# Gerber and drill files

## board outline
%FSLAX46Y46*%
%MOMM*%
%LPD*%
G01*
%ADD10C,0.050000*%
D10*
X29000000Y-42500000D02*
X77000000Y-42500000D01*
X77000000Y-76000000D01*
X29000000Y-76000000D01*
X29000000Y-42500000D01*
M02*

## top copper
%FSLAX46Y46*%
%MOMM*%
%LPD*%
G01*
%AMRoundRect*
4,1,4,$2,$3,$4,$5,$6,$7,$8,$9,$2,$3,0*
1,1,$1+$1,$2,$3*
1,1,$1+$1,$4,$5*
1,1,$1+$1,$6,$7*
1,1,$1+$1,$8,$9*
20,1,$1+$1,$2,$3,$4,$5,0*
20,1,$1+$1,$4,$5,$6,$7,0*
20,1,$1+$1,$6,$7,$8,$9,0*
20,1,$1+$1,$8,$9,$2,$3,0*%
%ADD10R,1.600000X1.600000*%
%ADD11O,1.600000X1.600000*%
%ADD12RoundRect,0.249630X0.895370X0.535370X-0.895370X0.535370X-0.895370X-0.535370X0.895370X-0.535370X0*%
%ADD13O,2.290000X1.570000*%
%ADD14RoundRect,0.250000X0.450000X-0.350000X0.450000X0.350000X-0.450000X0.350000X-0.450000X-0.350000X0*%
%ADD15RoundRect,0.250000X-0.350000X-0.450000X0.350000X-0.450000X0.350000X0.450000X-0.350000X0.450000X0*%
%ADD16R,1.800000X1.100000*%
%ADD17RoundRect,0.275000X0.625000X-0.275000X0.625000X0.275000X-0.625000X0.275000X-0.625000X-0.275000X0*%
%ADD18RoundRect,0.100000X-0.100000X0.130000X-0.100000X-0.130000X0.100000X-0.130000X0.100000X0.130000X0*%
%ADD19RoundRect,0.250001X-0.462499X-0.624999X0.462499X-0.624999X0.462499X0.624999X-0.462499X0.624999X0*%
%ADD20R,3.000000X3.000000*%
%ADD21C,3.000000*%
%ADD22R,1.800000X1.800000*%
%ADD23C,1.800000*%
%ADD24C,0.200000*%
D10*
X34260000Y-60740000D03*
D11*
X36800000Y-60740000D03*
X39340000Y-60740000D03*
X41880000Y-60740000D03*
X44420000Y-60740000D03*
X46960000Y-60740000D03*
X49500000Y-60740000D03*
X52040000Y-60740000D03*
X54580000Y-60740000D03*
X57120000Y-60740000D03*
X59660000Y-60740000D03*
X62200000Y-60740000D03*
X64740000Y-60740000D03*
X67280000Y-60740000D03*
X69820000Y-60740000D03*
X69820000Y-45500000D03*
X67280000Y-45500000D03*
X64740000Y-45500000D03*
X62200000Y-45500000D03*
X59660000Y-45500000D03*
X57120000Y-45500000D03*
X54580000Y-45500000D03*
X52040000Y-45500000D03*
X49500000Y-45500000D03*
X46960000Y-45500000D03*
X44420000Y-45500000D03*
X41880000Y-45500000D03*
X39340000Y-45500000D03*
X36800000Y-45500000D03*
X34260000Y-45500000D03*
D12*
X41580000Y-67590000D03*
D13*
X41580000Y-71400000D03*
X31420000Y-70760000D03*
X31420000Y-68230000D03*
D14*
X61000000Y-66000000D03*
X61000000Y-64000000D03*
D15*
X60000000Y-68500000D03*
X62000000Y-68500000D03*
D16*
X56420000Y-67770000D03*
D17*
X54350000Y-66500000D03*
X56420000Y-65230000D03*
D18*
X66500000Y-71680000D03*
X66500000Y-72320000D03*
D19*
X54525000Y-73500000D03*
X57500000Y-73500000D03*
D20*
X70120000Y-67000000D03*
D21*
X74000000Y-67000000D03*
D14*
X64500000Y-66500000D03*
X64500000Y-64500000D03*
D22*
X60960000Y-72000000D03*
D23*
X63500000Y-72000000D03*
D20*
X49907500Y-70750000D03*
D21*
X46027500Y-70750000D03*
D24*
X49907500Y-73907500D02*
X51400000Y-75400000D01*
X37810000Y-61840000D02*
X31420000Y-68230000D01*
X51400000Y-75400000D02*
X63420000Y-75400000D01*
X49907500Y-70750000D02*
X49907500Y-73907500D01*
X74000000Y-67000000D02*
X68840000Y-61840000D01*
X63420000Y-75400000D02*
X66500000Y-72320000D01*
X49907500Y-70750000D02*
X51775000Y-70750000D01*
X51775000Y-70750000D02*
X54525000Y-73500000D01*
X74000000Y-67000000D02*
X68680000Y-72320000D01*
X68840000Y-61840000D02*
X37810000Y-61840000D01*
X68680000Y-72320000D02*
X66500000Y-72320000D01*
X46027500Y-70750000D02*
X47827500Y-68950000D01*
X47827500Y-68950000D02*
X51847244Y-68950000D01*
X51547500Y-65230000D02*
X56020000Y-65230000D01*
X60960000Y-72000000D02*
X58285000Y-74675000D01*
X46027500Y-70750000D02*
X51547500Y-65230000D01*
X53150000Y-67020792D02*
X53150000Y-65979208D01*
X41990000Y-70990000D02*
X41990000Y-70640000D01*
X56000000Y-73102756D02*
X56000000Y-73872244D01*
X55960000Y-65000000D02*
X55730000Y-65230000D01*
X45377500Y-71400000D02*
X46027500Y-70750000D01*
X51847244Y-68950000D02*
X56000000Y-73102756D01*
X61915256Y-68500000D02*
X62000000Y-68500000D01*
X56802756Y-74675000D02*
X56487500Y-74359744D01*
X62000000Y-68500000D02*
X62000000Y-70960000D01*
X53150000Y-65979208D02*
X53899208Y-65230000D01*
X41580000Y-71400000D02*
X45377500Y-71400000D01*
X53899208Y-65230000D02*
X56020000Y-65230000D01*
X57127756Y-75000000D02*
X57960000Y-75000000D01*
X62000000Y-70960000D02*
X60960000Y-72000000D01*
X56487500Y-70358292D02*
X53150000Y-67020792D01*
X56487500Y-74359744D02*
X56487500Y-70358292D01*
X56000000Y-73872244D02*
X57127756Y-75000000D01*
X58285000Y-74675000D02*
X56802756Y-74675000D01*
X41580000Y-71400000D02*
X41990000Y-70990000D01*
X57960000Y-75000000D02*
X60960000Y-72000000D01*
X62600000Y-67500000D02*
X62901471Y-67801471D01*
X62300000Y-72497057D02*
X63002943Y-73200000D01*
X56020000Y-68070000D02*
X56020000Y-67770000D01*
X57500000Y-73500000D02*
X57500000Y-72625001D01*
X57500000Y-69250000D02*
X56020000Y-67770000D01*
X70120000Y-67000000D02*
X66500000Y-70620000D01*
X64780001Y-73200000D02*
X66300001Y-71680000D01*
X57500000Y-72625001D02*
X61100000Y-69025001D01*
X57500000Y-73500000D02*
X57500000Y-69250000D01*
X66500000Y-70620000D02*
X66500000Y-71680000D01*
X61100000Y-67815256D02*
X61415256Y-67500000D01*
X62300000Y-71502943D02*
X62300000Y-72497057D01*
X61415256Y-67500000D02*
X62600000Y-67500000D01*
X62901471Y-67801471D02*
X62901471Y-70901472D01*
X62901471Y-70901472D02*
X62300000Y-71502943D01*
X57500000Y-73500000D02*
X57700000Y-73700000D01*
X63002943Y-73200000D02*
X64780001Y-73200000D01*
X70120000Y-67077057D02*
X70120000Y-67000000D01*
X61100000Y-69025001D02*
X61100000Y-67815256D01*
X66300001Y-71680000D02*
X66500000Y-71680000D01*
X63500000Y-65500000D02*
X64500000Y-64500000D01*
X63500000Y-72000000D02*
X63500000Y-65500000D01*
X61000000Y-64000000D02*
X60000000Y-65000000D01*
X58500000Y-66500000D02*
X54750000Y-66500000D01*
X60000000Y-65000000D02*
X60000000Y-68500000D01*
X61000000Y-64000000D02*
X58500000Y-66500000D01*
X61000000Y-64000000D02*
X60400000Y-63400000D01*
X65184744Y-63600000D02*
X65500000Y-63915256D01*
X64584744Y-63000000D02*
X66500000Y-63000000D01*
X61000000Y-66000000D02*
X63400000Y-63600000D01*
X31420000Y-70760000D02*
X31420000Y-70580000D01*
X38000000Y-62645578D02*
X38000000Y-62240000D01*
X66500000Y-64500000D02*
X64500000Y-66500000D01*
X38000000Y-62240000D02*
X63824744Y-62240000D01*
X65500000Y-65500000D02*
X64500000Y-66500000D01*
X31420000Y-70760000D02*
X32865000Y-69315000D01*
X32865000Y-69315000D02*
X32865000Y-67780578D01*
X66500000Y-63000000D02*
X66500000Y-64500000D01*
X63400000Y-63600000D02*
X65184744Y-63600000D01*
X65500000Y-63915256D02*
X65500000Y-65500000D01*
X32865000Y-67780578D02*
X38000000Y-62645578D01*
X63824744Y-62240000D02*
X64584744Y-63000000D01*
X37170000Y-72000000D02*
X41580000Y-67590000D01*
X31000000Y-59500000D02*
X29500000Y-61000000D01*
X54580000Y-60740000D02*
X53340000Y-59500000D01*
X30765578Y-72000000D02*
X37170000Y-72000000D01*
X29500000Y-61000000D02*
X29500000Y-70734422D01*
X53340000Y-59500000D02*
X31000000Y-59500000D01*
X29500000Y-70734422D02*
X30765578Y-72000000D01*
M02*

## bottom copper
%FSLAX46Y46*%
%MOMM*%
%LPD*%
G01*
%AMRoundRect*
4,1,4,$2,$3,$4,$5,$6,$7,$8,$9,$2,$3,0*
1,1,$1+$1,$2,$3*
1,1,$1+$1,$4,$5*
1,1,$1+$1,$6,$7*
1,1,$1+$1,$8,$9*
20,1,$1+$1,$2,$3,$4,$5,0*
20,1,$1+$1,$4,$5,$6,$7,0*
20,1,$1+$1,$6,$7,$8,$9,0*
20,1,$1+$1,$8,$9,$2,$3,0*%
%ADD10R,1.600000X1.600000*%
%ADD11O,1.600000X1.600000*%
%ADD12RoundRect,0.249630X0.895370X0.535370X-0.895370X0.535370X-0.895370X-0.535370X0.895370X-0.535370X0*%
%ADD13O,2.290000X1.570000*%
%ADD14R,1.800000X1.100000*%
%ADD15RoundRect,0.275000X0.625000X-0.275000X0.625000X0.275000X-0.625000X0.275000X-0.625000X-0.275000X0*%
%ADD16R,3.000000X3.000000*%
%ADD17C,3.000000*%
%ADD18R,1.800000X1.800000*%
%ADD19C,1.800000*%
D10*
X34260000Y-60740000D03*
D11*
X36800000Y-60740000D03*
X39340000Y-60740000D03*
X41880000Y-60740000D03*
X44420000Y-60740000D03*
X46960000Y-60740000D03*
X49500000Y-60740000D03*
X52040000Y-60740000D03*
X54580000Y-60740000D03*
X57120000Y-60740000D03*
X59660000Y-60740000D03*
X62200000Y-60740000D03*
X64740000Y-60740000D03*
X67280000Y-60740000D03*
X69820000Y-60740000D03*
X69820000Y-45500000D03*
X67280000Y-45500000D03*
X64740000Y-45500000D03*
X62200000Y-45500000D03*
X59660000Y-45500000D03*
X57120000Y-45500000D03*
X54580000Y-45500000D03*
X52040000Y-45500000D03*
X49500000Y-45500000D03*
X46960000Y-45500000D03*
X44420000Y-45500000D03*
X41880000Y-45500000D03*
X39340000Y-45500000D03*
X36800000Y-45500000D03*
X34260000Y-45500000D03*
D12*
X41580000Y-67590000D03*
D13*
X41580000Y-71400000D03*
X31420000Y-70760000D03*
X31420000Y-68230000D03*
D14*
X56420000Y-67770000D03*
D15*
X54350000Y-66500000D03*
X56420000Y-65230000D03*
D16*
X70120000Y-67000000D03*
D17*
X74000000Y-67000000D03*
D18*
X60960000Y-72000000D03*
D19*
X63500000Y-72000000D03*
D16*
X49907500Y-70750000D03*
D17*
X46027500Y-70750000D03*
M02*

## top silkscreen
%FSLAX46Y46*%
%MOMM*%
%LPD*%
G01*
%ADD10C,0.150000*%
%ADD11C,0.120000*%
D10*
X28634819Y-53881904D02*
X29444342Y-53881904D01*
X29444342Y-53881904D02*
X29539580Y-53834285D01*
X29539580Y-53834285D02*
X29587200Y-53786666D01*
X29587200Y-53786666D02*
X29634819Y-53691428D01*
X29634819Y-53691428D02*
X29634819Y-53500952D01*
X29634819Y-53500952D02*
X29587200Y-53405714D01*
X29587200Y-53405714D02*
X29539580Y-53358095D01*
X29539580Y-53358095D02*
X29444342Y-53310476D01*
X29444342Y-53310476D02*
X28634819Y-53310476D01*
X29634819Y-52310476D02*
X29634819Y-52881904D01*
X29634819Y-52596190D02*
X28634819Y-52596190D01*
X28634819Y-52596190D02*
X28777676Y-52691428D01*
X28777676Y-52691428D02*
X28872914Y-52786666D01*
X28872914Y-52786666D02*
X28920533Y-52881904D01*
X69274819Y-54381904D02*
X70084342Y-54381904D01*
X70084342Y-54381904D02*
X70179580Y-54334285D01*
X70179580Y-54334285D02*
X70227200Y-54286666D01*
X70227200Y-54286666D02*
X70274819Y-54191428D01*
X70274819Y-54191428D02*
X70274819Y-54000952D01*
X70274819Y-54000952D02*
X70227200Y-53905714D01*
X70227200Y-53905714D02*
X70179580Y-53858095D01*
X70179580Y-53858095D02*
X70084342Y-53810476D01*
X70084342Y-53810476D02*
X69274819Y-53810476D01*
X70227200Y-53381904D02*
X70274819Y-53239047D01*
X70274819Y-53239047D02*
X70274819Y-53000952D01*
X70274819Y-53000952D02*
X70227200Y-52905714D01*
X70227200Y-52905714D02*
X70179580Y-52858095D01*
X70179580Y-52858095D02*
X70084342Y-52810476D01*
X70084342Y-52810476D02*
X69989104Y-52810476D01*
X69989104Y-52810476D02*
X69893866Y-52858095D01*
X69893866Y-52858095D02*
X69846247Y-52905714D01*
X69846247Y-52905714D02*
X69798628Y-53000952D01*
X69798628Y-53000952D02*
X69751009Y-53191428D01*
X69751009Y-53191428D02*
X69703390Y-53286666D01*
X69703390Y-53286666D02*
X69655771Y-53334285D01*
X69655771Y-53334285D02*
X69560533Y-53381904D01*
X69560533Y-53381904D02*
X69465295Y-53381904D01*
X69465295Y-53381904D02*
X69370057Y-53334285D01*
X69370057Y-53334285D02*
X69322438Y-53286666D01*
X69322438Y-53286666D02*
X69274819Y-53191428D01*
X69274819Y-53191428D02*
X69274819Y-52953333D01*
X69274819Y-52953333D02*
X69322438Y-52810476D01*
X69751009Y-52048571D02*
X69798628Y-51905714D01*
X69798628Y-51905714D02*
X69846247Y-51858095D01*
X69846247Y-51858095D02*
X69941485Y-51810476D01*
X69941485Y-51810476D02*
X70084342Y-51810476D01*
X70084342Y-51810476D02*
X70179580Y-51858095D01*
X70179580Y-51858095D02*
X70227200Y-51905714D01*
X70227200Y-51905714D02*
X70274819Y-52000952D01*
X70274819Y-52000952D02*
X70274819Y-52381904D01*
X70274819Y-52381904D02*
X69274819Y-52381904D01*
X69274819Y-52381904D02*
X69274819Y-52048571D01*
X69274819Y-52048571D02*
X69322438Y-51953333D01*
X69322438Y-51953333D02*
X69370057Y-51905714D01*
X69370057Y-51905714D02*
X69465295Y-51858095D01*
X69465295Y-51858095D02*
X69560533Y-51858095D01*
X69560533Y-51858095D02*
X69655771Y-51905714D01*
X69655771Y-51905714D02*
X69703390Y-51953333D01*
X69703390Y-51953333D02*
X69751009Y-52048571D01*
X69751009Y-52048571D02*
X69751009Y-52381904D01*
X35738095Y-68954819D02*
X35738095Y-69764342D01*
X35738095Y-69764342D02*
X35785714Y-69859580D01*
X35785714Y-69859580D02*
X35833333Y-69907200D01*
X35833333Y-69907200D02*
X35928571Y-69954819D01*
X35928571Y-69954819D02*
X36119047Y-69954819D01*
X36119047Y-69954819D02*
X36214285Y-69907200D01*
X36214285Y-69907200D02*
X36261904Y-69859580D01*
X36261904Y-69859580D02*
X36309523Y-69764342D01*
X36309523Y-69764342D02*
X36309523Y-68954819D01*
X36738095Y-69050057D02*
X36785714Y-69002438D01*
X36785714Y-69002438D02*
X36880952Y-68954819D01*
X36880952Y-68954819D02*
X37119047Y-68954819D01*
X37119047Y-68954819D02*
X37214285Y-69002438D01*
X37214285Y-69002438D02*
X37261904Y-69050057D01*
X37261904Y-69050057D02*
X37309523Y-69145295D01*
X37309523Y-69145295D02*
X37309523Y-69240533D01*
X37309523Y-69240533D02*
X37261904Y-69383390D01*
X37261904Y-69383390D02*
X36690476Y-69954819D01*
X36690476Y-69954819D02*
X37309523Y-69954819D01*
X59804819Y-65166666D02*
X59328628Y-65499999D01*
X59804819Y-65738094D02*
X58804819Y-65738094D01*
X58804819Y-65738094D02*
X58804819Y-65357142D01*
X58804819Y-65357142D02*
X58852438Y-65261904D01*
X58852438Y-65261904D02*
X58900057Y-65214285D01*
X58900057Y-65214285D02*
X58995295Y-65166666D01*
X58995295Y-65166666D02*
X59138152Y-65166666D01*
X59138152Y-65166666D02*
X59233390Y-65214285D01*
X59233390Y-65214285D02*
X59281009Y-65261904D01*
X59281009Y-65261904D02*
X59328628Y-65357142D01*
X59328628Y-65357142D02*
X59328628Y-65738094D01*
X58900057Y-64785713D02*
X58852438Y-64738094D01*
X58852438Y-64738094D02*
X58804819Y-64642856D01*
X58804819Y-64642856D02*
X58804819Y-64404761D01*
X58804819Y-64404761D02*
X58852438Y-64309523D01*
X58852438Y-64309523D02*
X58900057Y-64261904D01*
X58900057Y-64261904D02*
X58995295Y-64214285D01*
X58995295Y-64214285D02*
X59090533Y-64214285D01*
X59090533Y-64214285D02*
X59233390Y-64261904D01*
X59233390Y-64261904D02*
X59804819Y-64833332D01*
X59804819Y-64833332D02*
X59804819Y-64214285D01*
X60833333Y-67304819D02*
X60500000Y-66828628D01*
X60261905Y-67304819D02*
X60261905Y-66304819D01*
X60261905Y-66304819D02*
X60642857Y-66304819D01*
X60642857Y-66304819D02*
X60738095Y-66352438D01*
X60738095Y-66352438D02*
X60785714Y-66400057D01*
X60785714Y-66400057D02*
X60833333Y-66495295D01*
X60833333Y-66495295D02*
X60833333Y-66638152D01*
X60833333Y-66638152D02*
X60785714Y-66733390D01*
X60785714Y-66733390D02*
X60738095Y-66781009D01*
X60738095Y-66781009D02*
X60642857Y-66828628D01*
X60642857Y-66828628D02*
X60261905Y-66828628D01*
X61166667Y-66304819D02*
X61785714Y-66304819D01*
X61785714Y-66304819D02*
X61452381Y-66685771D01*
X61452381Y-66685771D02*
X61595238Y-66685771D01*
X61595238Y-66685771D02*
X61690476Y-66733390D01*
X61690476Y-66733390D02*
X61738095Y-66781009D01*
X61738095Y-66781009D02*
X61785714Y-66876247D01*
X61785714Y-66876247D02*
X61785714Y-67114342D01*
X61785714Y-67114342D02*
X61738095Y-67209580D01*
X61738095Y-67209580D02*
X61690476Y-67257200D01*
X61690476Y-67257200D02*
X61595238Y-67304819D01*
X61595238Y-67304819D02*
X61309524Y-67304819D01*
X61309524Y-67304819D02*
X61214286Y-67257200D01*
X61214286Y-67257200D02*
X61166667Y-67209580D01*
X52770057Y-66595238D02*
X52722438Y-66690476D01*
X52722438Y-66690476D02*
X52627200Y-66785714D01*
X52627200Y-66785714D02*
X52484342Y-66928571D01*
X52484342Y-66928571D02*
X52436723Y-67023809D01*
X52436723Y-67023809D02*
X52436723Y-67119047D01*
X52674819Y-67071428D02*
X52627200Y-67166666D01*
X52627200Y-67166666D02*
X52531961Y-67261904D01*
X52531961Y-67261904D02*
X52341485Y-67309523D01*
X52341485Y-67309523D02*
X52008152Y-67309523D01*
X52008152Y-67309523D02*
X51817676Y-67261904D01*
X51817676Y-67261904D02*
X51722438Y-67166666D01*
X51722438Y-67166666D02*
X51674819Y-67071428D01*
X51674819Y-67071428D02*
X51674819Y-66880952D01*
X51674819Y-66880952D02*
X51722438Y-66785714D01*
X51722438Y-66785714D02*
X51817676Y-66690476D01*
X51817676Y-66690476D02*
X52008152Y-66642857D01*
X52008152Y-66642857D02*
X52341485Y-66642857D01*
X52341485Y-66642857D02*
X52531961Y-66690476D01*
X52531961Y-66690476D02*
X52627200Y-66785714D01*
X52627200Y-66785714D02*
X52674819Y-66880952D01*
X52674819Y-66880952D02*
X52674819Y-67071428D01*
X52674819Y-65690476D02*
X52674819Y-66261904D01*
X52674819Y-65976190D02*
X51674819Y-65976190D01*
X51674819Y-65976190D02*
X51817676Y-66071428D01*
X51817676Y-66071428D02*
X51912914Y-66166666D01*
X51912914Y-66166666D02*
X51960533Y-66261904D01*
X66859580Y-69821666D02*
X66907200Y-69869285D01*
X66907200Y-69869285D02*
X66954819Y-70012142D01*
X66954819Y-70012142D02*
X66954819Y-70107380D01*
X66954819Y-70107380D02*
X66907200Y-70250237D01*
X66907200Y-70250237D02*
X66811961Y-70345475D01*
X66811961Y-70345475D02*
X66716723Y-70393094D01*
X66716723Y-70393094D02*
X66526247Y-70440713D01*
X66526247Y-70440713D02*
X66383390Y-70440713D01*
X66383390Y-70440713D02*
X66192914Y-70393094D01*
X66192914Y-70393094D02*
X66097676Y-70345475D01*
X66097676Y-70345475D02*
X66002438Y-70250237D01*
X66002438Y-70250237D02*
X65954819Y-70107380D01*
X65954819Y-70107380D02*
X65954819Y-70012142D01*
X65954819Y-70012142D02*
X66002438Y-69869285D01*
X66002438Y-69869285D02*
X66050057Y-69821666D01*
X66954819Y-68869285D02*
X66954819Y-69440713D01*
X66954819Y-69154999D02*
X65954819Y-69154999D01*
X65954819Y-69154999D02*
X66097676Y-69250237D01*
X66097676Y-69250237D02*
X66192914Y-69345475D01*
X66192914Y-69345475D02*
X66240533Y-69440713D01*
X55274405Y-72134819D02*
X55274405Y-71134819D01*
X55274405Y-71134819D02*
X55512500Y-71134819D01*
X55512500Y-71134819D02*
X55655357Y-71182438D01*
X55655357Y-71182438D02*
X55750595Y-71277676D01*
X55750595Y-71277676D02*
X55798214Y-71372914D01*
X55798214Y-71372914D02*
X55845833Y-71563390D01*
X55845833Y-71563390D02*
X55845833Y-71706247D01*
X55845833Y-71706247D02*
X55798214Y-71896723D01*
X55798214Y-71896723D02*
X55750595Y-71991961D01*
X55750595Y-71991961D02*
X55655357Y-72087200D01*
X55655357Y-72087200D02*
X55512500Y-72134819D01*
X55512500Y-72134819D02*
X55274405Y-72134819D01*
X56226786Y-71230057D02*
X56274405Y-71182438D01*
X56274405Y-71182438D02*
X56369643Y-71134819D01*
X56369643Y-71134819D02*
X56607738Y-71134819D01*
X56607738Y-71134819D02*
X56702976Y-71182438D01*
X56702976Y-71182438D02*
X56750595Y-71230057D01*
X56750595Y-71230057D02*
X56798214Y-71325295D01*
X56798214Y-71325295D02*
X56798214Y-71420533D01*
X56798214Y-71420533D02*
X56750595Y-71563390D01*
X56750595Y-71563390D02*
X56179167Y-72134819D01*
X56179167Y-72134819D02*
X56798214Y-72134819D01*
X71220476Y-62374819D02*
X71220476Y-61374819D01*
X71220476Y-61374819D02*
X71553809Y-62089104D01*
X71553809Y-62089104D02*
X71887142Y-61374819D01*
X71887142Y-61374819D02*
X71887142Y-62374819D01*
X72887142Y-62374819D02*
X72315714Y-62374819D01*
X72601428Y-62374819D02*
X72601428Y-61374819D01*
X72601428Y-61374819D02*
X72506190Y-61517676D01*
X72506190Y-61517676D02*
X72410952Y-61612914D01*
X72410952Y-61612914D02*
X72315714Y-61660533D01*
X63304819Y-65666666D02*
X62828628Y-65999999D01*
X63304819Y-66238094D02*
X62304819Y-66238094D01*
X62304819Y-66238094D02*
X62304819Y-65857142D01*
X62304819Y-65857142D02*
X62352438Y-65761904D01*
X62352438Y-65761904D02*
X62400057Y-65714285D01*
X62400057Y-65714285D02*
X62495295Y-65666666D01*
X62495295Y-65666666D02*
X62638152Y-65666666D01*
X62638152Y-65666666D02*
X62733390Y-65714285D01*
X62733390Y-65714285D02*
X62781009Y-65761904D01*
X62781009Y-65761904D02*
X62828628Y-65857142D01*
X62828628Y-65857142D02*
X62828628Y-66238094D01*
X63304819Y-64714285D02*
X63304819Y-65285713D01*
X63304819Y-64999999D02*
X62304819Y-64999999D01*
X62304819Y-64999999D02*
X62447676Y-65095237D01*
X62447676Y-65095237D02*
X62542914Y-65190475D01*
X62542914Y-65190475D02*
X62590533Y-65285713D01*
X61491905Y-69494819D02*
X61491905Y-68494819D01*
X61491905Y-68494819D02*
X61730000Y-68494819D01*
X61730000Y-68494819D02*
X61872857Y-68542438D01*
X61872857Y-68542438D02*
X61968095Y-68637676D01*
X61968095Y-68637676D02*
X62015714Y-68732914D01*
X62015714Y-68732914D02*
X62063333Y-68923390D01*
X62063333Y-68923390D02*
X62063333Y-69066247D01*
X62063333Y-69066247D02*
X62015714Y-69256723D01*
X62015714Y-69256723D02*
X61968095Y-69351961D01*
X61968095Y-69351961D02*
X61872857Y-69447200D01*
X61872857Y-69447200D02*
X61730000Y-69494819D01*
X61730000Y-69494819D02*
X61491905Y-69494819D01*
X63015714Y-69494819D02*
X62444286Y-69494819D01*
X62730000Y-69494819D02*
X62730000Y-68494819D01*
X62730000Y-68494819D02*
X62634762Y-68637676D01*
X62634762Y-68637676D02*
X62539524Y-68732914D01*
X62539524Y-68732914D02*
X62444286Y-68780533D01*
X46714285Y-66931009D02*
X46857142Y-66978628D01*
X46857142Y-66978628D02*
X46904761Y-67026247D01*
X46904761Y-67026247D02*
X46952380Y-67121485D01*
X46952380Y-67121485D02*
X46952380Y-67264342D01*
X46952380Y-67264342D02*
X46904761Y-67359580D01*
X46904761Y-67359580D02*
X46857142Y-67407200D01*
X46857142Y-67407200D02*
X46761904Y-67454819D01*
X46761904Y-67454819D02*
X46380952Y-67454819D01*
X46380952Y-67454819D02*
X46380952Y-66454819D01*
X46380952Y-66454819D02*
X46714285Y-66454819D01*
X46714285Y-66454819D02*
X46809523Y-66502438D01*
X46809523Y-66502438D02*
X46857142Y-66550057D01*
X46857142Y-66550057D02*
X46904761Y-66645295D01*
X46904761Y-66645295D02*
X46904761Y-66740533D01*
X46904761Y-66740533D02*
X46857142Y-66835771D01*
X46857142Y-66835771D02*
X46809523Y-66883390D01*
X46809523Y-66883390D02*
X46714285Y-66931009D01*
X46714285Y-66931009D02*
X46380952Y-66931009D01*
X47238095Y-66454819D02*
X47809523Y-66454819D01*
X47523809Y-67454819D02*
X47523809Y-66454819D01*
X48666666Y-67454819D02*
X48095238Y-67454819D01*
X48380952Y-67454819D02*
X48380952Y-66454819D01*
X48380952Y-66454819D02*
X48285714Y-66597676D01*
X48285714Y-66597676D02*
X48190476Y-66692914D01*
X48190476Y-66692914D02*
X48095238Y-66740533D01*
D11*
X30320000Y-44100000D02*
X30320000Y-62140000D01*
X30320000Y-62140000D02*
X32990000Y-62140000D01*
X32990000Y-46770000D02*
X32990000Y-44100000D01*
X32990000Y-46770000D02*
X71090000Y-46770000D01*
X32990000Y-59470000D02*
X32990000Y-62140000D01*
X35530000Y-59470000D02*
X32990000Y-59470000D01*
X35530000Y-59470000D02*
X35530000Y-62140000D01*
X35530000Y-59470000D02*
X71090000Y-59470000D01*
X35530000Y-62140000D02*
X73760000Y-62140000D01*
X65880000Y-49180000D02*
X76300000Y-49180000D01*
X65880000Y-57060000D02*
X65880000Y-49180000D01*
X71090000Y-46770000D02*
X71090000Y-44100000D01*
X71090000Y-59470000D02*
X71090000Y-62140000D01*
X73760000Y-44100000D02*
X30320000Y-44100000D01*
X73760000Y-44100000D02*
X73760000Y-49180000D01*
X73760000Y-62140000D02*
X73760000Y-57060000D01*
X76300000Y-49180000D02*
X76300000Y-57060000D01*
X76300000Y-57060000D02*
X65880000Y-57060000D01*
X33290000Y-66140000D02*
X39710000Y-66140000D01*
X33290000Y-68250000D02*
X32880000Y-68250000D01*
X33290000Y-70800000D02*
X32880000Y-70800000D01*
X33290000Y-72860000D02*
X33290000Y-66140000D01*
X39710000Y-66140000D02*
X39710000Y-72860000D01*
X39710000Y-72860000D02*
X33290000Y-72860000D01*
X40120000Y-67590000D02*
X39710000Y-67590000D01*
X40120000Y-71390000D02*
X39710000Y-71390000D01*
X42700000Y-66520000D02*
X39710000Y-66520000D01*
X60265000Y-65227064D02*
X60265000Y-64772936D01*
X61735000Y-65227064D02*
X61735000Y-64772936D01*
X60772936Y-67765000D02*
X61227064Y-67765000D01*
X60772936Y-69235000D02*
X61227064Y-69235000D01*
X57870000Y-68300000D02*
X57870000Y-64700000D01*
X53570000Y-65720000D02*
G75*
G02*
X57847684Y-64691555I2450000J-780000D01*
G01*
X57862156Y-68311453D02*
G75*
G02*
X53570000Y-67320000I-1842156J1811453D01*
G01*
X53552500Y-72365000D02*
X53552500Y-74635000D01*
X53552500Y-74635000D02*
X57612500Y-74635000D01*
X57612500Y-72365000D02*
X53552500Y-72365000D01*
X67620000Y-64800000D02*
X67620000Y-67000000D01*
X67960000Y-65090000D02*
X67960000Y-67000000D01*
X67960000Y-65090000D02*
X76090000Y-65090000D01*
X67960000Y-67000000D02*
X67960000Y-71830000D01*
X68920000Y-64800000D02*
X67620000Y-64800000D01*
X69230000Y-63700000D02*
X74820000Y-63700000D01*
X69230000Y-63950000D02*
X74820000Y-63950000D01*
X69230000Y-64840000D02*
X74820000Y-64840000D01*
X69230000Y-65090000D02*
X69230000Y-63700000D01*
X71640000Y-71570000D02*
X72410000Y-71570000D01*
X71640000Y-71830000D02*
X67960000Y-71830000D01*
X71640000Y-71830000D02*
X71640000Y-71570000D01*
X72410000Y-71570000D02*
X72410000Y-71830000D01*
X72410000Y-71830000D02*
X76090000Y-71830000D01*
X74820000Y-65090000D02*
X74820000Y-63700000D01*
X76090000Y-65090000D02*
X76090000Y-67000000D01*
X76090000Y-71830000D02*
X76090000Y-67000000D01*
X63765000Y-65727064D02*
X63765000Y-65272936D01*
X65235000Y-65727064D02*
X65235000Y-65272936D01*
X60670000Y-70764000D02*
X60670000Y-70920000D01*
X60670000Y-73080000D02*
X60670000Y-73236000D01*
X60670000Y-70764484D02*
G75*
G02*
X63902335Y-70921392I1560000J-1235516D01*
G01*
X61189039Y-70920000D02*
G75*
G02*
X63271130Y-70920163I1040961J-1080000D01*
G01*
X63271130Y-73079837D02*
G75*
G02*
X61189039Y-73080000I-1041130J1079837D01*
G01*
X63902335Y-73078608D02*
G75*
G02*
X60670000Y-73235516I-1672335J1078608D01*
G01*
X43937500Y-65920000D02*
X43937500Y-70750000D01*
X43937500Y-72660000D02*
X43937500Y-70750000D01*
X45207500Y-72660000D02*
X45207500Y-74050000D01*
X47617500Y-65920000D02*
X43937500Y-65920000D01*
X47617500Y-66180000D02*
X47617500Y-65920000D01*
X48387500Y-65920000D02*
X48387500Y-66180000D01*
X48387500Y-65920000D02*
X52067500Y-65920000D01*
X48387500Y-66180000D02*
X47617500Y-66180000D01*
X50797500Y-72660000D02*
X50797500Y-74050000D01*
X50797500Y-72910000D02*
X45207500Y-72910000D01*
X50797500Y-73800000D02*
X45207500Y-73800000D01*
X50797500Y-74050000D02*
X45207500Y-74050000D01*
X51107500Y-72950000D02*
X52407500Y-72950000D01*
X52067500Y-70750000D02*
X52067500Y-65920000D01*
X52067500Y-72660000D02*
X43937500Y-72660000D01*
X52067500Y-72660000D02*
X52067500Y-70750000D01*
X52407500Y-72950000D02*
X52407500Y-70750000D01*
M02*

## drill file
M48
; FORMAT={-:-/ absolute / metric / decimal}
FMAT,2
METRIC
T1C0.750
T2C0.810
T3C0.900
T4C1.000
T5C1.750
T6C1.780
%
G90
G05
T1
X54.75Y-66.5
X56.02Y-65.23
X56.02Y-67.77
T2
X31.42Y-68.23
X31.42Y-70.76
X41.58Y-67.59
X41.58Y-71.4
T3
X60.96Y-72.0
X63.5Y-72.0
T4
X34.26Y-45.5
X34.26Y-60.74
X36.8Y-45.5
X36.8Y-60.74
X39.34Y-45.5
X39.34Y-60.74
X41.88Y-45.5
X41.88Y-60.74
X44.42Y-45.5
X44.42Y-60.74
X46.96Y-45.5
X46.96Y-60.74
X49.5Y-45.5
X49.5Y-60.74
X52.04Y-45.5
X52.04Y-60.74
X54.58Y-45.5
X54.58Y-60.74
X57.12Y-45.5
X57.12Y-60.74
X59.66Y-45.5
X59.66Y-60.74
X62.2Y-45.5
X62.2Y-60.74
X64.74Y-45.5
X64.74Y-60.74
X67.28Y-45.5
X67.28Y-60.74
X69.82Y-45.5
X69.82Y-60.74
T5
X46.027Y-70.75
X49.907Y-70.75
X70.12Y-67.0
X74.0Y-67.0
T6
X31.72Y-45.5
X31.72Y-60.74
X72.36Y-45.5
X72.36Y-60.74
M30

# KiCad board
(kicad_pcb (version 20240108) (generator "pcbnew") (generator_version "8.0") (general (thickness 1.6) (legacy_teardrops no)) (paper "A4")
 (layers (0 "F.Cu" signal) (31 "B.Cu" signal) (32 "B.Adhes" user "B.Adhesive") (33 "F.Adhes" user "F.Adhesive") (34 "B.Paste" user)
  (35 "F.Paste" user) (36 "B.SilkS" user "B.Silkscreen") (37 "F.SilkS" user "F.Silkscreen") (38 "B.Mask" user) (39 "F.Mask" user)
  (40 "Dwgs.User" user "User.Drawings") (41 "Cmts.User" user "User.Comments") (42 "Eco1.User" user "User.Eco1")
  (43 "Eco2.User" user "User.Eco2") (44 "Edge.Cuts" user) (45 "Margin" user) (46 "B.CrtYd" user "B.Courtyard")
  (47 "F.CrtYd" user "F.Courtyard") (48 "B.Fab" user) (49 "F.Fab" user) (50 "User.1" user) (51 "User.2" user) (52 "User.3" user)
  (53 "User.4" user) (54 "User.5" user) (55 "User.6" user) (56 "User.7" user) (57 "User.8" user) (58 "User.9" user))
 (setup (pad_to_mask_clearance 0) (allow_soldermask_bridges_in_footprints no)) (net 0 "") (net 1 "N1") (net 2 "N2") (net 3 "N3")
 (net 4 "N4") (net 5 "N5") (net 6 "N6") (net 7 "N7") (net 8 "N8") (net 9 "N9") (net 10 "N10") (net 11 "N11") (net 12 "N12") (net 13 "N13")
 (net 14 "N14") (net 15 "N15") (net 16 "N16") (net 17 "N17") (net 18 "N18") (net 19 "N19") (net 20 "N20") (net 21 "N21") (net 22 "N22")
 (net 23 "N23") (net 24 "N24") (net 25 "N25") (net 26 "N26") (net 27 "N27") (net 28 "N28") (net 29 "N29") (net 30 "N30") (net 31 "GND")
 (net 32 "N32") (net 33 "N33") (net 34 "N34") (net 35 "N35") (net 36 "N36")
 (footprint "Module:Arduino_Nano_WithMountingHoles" (layer "F.Cu") (at 34.26 60.74 90)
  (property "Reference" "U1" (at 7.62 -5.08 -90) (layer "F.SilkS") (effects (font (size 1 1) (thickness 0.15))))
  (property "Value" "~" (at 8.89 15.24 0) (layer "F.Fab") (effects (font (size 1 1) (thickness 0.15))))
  (fp_line (start 16.64 -3.94) (end -1.4 -3.94) (stroke (width 0.12) (type solid)) (layer "F.SilkS"))
  (fp_line (start -1.4 -3.94) (end -1.4 -1.27) (stroke (width 0.12) (type solid)) (layer "F.SilkS"))
  (fp_line (start 13.97 -1.27) (end 16.64 -1.27) (stroke (width 0.12) (type solid)) (layer "F.SilkS"))
  (fp_line (start 13.97 -1.27) (end 13.97 36.83) (stroke (width 0.12) (type solid)) (layer "F.SilkS"))
  (fp_line (start 1.27 -1.27) (end -1.4 -1.27) (stroke (width 0.12) (type solid)) (layer "F.SilkS"))
  (fp_line (start 1.27 1.27) (end 1.27 -1.27) (stroke (width 0.12) (type solid)) (layer "F.SilkS"))
  (fp_line (start 1.27 1.27) (end -1.4 1.27) (stroke (width 0.12) (type solid)) (layer "F.SilkS"))
  (fp_line (start 1.27 1.27) (end 1.27 36.83) (stroke (width 0.12) (type solid)) (layer "F.SilkS"))
  (fp_line (start -1.4 1.27) (end -1.4 39.5) (stroke (width 0.12) (type solid)) (layer "F.SilkS"))
  (fp_line (start 11.56 31.62) (end 11.56 42.04) (stroke (width 0.12) (type solid)) (layer "F.SilkS"))
  (fp_line (start 3.68 31.62) (end 11.56 31.62) (stroke (width 0.12) (type solid)) (layer "F.SilkS"))
  (fp_line (start 13.97 36.83) (end 16.64 36.83) (stroke (width 0.12) (type solid)) (layer "F.SilkS"))
  (fp_line (start 1.27 36.83) (end -1.4 36.83) (stroke (width 0.12) (type solid)) (layer "F.SilkS"))
  (fp_line (start 16.64 39.5) (end 16.64 -3.94) (stroke (width 0.12) (type solid)) (layer "F.SilkS"))
  (fp_line (start 16.64 39.5) (end 11.56 39.5) (stroke (width 0.12) (type solid)) (layer "F.SilkS"))
  (fp_line (start -1.4 39.5) (end 3.68 39.5) (stroke (width 0.12) (type solid)) (layer "F.SilkS"))
  (fp_line (start 11.56 42.04) (end 3.68 42.04) (stroke (width 0.12) (type solid)) (layer "F.SilkS"))
  (fp_line (start 3.68 42.04) (end 3.68 31.62) (stroke (width 0.12) (type solid)) (layer "F.SilkS"))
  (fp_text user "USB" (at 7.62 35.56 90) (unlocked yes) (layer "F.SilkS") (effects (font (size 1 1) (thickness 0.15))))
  (pad "" np_thru_hole circle (at 0 -2.54 90) (size 1.78 1.78) (drill 1.78) (layers "*.Cu" "*.Mask"))
  (pad "" np_thru_hole circle (at 0 38.1 90) (size 1.78 1.78) (drill 1.78) (layers "*.Cu" "*.Mask"))
  (pad "" np_thru_hole circle (at 15.24 -2.54 90) (size 1.78 1.78) (drill 1.78) (layers "*.Cu" "*.Mask"))
  (pad "" np_thru_hole circle (at 15.24 38.1 90) (size 1.78 1.78) (drill 1.78) (layers "*.Cu" "*.Mask"))
  (pad "1" thru_hole rect (at 0 0 90) (size 1.6 1.6) (drill 1) (layers "*.Cu" "*.Mask") (remove_unused_layers no) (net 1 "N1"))
  (pad "2" thru_hole oval (at 0 2.54 90) (size 1.6 1.6) (drill 1) (layers "*.Cu" "*.Mask") (remove_unused_layers no) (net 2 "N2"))
  (pad "3" thru_hole oval (at 0 5.08 90) (size 1.6 1.6) (drill 1) (layers "*.Cu" "*.Mask") (remove_unused_layers no) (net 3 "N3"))
  (pad "4" thru_hole oval (at 0 7.62 90) (size 1.6 1.6) (drill 1) (layers "*.Cu" "*.Mask") (remove_unused_layers no) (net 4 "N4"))
  (pad "5" thru_hole oval (at 0 10.16 90) (size 1.6 1.6) (drill 1) (layers "*.Cu" "*.Mask") (remove_unused_layers no) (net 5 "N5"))
  (pad "6" thru_hole oval (at 0 12.7 90) (size 1.6 1.6) (drill 1) (layers "*.Cu" "*.Mask") (remove_unused_layers no) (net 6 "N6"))
  (pad "7" thru_hole oval (at 0 15.24 90) (size 1.6 1.6) (drill 1) (layers "*.Cu" "*.Mask") (remove_unused_layers no) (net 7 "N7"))
  (pad "8" thru_hole oval (at 0 17.78 90) (size 1.6 1.6) (drill 1) (layers "*.Cu" "*.Mask") (remove_unused_layers no) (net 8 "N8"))
  (pad "9" thru_hole oval (at 0 20.32 90) (size 1.6 1.6) (drill 1) (layers "*.Cu" "*.Mask") (remove_unused_layers no) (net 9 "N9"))
  (pad "10" thru_hole oval (at 0 22.86 90) (size 1.6 1.6) (drill 1) (layers "*.Cu" "*.Mask") (remove_unused_layers no) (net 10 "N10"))
  (pad "11" thru_hole oval (at 0 25.4 90) (size 1.6 1.6) (drill 1) (layers "*.Cu" "*.Mask") (remove_unused_layers no) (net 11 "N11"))
  (pad "12" thru_hole oval (at 0 27.94 90) (size 1.6 1.6) (drill 1) (layers "*.Cu" "*.Mask") (remove_unused_layers no) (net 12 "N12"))
  (pad "13" thru_hole oval (at 0 30.48 90) (size 1.6 1.6) (drill 1) (layers "*.Cu" "*.Mask") (remove_unused_layers no) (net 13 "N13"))
  (pad "14" thru_hole oval (at 0 33.02 90) (size 1.6 1.6) (drill 1) (layers "*.Cu" "*.Mask") (remove_unused_layers no) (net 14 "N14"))
  (pad "15" thru_hole oval (at 0 35.56 90) (size 1.6 1.6) (drill 1) (layers "*.Cu" "*.Mask") (remove_unused_layers no) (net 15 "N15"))
  (pad "16" thru_hole oval (at 15.24 35.56 90) (size 1.6 1.6) (drill 1) (layers "*.Cu" "*.Mask") (remove_unused_layers no) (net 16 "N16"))
  (pad "17" thru_hole oval (at 15.24 33.02 90) (size 1.6 1.6) (drill 1) (layers "*.Cu" "*.Mask") (remove_unused_layers no) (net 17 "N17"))
  (pad "18" thru_hole oval (at 15.24 30.48 90) (size 1.6 1.6) (drill 1) (layers "*.Cu" "*.Mask") (remove_unused_layers no) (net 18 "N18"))
  (pad "19" thru_hole oval (at 15.24 27.94 90) (size 1.6 1.6) (drill 1) (layers "*.Cu" "*.Mask") (remove_unused_layers no) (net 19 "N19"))
  (pad "20" thru_hole oval (at 15.24 25.4 90) (size 1.6 1.6) (drill 1) (layers "*.Cu" "*.Mask") (remove_unused_layers no) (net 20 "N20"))
  (pad "21" thru_hole oval (at 15.24 22.86 90) (size 1.6 1.6) (drill 1) (layers "*.Cu" "*.Mask") (remove_unused_layers no) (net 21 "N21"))
  (pad "22" thru_hole oval (at 15.24 20.32 90) (size 1.6 1.6) (drill 1) (layers "*.Cu" "*.Mask") (remove_unused_layers no) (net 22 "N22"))
  (pad "23" thru_hole oval (at 15.24 17.78 90) (size 1.6 1.6) (drill 1) (layers "*.Cu" "*.Mask") (remove_unused_layers no) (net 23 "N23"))
  (pad "24" thru_hole oval (at 15.24 15.24 90) (size 1.6 1.6) (drill 1) (layers "*.Cu" "*.Mask") (remove_unused_layers no) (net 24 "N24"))
  (pad "25" thru_hole oval (at 15.24 12.7 90) (size 1.6 1.6) (drill 1) (layers "*.Cu" "*.Mask") (remove_unused_layers no) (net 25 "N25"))
  (pad "26" thru_hole oval (at 15.24 10.16 90) (size 1.6 1.6) (drill 1) (layers "*.Cu" "*.Mask") (remove_unused_layers no) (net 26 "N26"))
  (pad "27" thru_hole oval (at 15.24 7.62 90) (size 1.6 1.6) (drill 1) (layers "*.Cu" "*.Mask") (remove_unused_layers no) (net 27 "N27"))
  (pad "28" thru_hole oval (at 15.24 5.08 90) (size 1.6 1.6) (drill 1) (layers "*.Cu" "*.Mask") (remove_unused_layers no) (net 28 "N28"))
  (pad "29" thru_hole oval (at 15.24 2.54 90) (size 1.6 1.6) (drill 1) (layers "*.Cu" "*.Mask") (remove_unused_layers no) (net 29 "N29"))
  (pad "30" thru_hole oval (at 15.24 0 90) (size 1.6 1.6) (drill 1) (layers "*.Cu" "*.Mask") (remove_unused_layers no) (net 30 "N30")))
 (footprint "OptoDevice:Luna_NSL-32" (layer "F.Cu") (at 41.58 67.59 180)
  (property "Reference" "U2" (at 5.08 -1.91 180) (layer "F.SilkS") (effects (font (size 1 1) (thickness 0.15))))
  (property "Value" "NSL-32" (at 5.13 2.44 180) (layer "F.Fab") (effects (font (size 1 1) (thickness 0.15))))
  (fp_line (start 8.29 1.45) (end 1.87 1.45) (stroke (width 0.12) (type solid)) (layer "F.SilkS"))
  (fp_line (start 8.29 -0.66) (end 8.7 -0.66) (stroke (width 0.12) (type solid)) (layer "F.SilkS"))
  (fp_line (start 8.29 -3.21) (end 8.7 -3.21) (stroke (width 0.12) (type solid)) (layer "F.SilkS"))
  (fp_line (start 8.29 -5.27) (end 8.29 1.45) (stroke (width 0.12) (type solid)) (layer "F.SilkS"))
  (fp_line (start 1.87 1.45) (end 1.87 -5.27) (stroke (width 0.12) (type solid)) (layer "F.SilkS"))
  (fp_line (start 1.87 -5.27) (end 8.29 -5.27) (stroke (width 0.12) (type solid)) (layer "F.SilkS"))
  (fp_line (start 1.46 0) (end 1.87 0) (stroke (width 0.12) (type solid)) (layer "F.SilkS"))
  (fp_line (start 1.46 -3.8) (end 1.87 -3.8) (stroke (width 0.12) (type solid)) (layer "F.SilkS"))
  (fp_line (start -1.12 1.07) (end 1.87 1.07) (stroke (width 0.12) (type solid)) (layer "F.SilkS"))
  (pad "1" thru_hole roundrect (at 0 0 180) (size 2.29 1.57) (drill 0.81) (layers "*.Cu" "*.Mask") (remove_unused_layers no)
   (roundrect_rratio 0.159) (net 9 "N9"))
  (pad "2" thru_hole oval (at 0 -3.81 180) (size 2.29 1.57) (drill 0.81) (layers "*.Cu" "*.Mask") (remove_unused_layers no) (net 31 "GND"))
  (pad "3" thru_hole oval (at 10.16 -3.17 180) (size 2.29 1.57) (drill 0.81) (layers "*.Cu" "*.Mask") (remove_unused_layers no)
   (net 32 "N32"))
  (pad "4" thru_hole oval (at 10.16 -0.64 180) (size 2.29 1.57) (drill 0.81) (layers "*.Cu" "*.Mask") (remove_unused_layers no)
   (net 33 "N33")))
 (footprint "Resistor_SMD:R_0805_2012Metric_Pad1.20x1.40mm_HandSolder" (layer "F.Cu") (at 61 65 90)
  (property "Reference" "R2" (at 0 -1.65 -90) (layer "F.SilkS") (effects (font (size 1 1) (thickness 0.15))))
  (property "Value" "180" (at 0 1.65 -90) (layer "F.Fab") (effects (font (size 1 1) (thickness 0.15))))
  (fp_line (start -0.227064 -0.735) (end 0.227064 -0.735) (stroke (width 0.12) (type solid)) (layer "F.SilkS"))
  (fp_line (start -0.227064 0.735) (end 0.227064 0.735) (stroke (width 0.12) (type solid)) (layer "F.SilkS"))
  (pad "1" smd roundrect (at -1 0 90) (size 1.2 1.4) (layers "F.Cu" "F.Paste" "F.Mask") (roundrect_rratio 0.208333) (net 32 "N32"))
  (pad "2" smd roundrect (at 1 0 90) (size 1.2 1.4) (layers "F.Cu" "F.Paste" "F.Mask") (roundrect_rratio 0.208333) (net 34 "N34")))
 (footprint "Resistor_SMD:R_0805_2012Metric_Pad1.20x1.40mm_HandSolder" (layer "F.Cu") (at 61 68.5)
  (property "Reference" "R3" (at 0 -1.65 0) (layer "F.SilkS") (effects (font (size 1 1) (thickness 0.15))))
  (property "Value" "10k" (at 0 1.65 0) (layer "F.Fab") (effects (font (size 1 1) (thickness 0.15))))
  (fp_line (start -0.227064 -0.735) (end 0.227064 -0.735) (stroke (width 0.12) (type solid)) (layer "F.SilkS"))
  (fp_line (start -0.227064 0.735) (end 0.227064 0.735) (stroke (width 0.12) (type solid)) (layer "F.SilkS"))
  (pad "1" smd roundrect (at -1 0) (size 1.2 1.4) (layers "F.Cu" "F.Paste" "F.Mask") (roundrect_rratio 0.208333) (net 34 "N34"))
  (pad "2" smd roundrect (at 1 0) (size 1.2 1.4) (layers "F.Cu" "F.Paste" "F.Mask") (roundrect_rratio 0.208333) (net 31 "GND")))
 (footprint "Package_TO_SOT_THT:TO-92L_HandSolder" (layer "F.Cu") (at 56.02 67.77 90)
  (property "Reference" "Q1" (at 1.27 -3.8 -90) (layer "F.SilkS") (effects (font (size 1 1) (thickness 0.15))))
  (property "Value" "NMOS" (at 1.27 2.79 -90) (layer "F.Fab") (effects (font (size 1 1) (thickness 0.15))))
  (fp_line (start -0.53 1.85) (end 3.07 1.85) (stroke (width 0.12) (type solid)) (layer "F.SilkS"))
  (fp_arc (start 2.05 -2.45) (mid 3.769931 -0.601036) (end 3.078445 1.827684) (stroke (width 0.12) (type solid)) (layer "F.SilkS"))
  (fp_arc (start -0.541453 1.842156) (mid -1.247298 -0.581475) (end 0.45 -2.45) (stroke (width 0.12) (type solid)) (layer "F.SilkS"))
  (pad "1" thru_hole rect (at 0 0 90) (size 1.1 1.8) (drill 0.75 (offset 0 0.4)) (layers "*.Cu" "*.Mask") (remove_unused_layers no)
   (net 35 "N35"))
  (pad "2" thru_hole roundrect (at 1.27 -1.27 90) (size 1.1 1.8) (drill 0.75 (offset 0 -0.4)) (layers "*.Cu" "*.Mask")
   (remove_unused_layers no) (roundrect_rratio 0.25) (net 34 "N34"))
  (pad "3" thru_hole roundrect (at 2.54 0 90) (size 1.1 1.8) (drill 0.75 (offset 0 0.4)) (layers "*.Cu" "*.Mask") (remove_unused_layers no)
   (roundrect_rratio 0.25) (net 31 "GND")))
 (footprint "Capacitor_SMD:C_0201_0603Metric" (layer "F.Cu") (at 66.5 72 -90)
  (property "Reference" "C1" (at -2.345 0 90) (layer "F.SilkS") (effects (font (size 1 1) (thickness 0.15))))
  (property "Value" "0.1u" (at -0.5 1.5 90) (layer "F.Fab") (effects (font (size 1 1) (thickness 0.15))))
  (pad "" smd roundrect (at -0.345 0 270) (size 0.318 0.36) (layers "F.Paste") (roundrect_rratio 0.25))
  (pad "" smd roundrect (at 0.345 0 270) (size 0.318 0.36) (layers "F.Paste") (roundrect_rratio 0.25))
  (pad "1" smd roundrect (at -0.32 0 270) (size 0.46 0.4) (layers "F.Cu" "F.Mask") (roundrect_rratio 0.25) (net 35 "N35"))
  (pad "2" smd roundrect (at 0.32 0 270) (size 0.46 0.4) (layers "F.Cu" "F.Mask") (roundrect_rratio 0.25) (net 33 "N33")))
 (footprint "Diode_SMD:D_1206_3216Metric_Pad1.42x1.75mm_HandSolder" (layer "F.Cu") (at 56.0125 73.5)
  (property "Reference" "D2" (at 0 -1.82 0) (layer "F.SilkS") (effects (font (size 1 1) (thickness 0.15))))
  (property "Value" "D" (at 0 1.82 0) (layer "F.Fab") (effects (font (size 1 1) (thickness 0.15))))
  (fp_line (start -2.46 -1.135) (end -2.46 1.135) (stroke (width 0.12) (type solid)) (layer "F.SilkS"))
  (fp_line (start -2.46 1.135) (end 1.6 1.135) (stroke (width 0.12) (type solid)) (layer "F.SilkS"))
  (fp_line (start 1.6 -1.135) (end -2.46 -1.135) (stroke (width 0.12) (type solid)) (layer "F.SilkS"))
  (pad "1" smd roundrect (at -1.4875 0) (size 1.425 1.75) (layers "F.Cu" "F.Paste" "F.Mask") (roundrect_rratio 0.175439) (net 33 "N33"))
  (pad "2" smd roundrect (at 1.4875 0) (size 1.425 1.75) (layers "F.Cu" "F.Paste" "F.Mask") (roundrect_rratio 0.175439) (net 35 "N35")))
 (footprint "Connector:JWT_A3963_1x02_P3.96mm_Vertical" (layer "F.Cu") (at 70.12 67)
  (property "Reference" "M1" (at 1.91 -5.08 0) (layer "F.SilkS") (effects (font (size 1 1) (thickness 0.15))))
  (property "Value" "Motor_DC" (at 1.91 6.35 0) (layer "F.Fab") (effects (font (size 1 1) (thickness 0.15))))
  (fp_line (start -2.5 -2.2) (end -2.5 0) (stroke (width 0.12) (type solid)) (layer "F.SilkS"))
  (fp_line (start -2.16 -1.91) (end -2.16 0) (stroke (width 0.12) (type solid)) (layer "F.SilkS"))
  (fp_line (start -2.16 -1.91) (end 5.97 -1.91) (stroke (width 0.12) (type solid)) (layer "F.SilkS"))
  (fp_line (start -2.16 0) (end -2.16 4.83) (stroke (width 0.12) (type solid)) (layer "F.SilkS"))
  (fp_line (start -1.2 -2.2) (end -2.5 -2.2) (stroke (width 0.12) (type solid)) (layer "F.SilkS"))
  (fp_line (start -0.89 -3.3) (end 4.7 -3.3) (stroke (width 0.12) (type solid)) (layer "F.SilkS"))
  (fp_line (start -0.89 -3.05) (end 4.7 -3.05) (stroke (width 0.12) (type solid)) (layer "F.SilkS"))
  (fp_line (start -0.89 -2.16) (end 4.7 -2.16) (stroke (width 0.12) (type solid)) (layer "F.SilkS"))
  (fp_line (start -0.89 -1.91) (end -0.89 -3.3) (stroke (width 0.12) (type solid)) (layer "F.SilkS"))
  (fp_line (start 1.52 4.57) (end 2.29 4.57) (stroke (width 0.12) (type solid)) (layer "F.SilkS"))
  (fp_line (start 1.52 4.83) (end -2.16 4.83) (stroke (width 0.12) (type solid)) (layer "F.SilkS"))
  (fp_line (start 1.52 4.83) (end 1.52 4.57) (stroke (width 0.12) (type solid)) (layer "F.SilkS"))
  (fp_line (start 2.29 4.57) (end 2.29 4.83) (stroke (width 0.12) (type solid)) (layer "F.SilkS"))
  (fp_line (start 2.29 4.83) (end 5.97 4.83) (stroke (width 0.12) (type solid)) (layer "F.SilkS"))
  (fp_line (start 4.7 -1.91) (end 4.7 -3.3) (stroke (width 0.12) (type solid)) (layer "F.SilkS"))
  (fp_line (start 5.97 -1.91) (end 5.97 0) (stroke (width 0.12) (type solid)) (layer "F.SilkS"))
  (fp_line (start 5.97 4.83) (end 5.97 0) (stroke (width 0.12) (type solid)) (layer "F.SilkS"))
  (pad "1" thru_hole rect (at 0 0) (size 3 3) (drill 1.75) (layers "*.Cu" "*.Mask") (remove_unused_layers no) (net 35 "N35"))
  (pad "2" thru_hole circle (at 3.88 0) (size 3 3) (drill 1.75) (layers "*.Cu" "*.Mask") (remove_unused_layers no) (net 33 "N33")))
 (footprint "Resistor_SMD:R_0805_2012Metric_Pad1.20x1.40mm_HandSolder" (layer "F.Cu") (at 64.5 65.5 90)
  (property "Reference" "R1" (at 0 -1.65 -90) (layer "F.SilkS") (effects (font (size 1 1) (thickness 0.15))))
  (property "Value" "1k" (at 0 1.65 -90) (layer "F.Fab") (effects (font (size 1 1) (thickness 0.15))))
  (fp_line (start -0.227064 -0.735) (end 0.227064 -0.735) (stroke (width 0.12) (type solid)) (layer "F.SilkS"))
  (fp_line (start -0.227064 0.735) (end 0.227064 0.735) (stroke (width 0.12) (type solid)) (layer "F.SilkS"))
  (pad "1" smd roundrect (at -1 0 90) (size 1.2 1.4) (layers "F.Cu" "F.Paste" "F.Mask") (roundrect_rratio 0.208333) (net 32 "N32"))
  (pad "2" smd roundrect (at 1 0 90) (size 1.2 1.4) (layers "F.Cu" "F.Paste" "F.Mask") (roundrect_rratio 0.208333) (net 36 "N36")))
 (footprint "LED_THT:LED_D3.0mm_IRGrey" (layer "F.Cu") (at 60.96 72)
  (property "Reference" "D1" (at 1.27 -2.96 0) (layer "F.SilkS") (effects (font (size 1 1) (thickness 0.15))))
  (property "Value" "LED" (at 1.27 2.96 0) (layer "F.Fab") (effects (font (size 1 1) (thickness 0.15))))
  (fp_line (start -0.29 -1.236) (end -0.29 -1.08) (stroke (width 0.12) (type solid)) (layer "F.SilkS"))
  (fp_line (start -0.29 1.08) (end -0.29 1.236) (stroke (width 0.12) (type solid)) (layer "F.SilkS"))
  (fp_arc (start -0.29 -1.235516) (mid 1.366487 -1.987659) (end 2.942335 -1.078608) (stroke (width 0.12) (type solid)) (layer "F.SilkS"))
  (fp_arc (start 0.229039 -1.08) (mid 1.270117 -1.5) (end 2.31113 -1.079837) (stroke (width 0.12) (type solid)) (layer "F.SilkS"))
  (fp_arc (start 2.31113 1.079837) (mid 1.270117 1.5) (end 0.229039 1.08) (stroke (width 0.12) (type solid)) (layer "F.SilkS"))
  (fp_arc (start 2.942335 1.078608) (mid 1.366487 1.987659) (end -0.29 1.235516) (stroke (width 0.12) (type solid)) (layer "F.SilkS"))
  (pad "1" thru_hole rect (at 0 0) (size 1.8 1.8) (drill 0.9) (layers "*.Cu" "*.Mask") (remove_unused_layers no) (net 31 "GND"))
  (pad "2" thru_hole circle (at 2.54 0) (size 1.8 1.8) (drill 0.9) (layers "*.Cu" "*.Mask") (remove_unused_layers no) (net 36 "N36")))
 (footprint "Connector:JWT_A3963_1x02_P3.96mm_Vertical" (layer "F.Cu") (at 49.9075 70.75 180)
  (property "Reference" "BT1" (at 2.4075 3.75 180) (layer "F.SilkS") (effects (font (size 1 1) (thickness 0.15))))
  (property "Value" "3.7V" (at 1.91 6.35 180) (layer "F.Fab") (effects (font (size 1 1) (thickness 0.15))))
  (fp_line (start 5.97 4.83) (end 5.97 0) (stroke (width 0.12) (type solid)) (layer "F.SilkS"))
  (fp_line (start 5.97 -1.91) (end 5.97 0) (stroke (width 0.12) (type solid)) (layer "F.SilkS"))
  (fp_line (start 4.7 -1.91) (end 4.7 -3.3) (stroke (width 0.12) (type solid)) (layer "F.SilkS"))
  (fp_line (start 2.29 4.83) (end 5.97 4.83) (stroke (width 0.12) (type solid)) (layer "F.SilkS"))
  (fp_line (start 2.29 4.57) (end 2.29 4.83) (stroke (width 0.12) (type solid)) (layer "F.SilkS"))
  (fp_line (start 1.52 4.83) (end 1.52 4.57) (stroke (width 0.12) (type solid)) (layer "F.SilkS"))
  (fp_line (start 1.52 4.83) (end -2.16 4.83) (stroke (width 0.12) (type solid)) (layer "F.SilkS"))
  (fp_line (start 1.52 4.57) (end 2.29 4.57) (stroke (width 0.12) (type solid)) (layer "F.SilkS"))
  (fp_line (start -0.89 -1.91) (end -0.89 -3.3) (stroke (width 0.12) (type solid)) (layer "F.SilkS"))
  (fp_line (start -0.89 -2.16) (end 4.7 -2.16) (stroke (width 0.12) (type solid)) (layer "F.SilkS"))
  (fp_line (start -0.89 -3.05) (end 4.7 -3.05) (stroke (width 0.12) (type solid)) (layer "F.SilkS"))
  (fp_line (start -0.89 -3.3) (end 4.7 -3.3) (stroke (width 0.12) (type solid)) (layer "F.SilkS"))
  (fp_line (start -1.2 -2.2) (end -2.5 -2.2) (stroke (width 0.12) (type solid)) (layer "F.SilkS"))
  (fp_line (start -2.16 0) (end -2.16 4.83) (stroke (width 0.12) (type solid)) (layer "F.SilkS"))
  (fp_line (start -2.16 -1.91) (end 5.97 -1.91) (stroke (width 0.12) (type solid)) (layer "F.SilkS"))
  (fp_line (start -2.16 -1.91) (end -2.16 0) (stroke (width 0.12) (type solid)) (layer "F.SilkS"))
  (fp_line (start -2.5 -2.2) (end -2.5 0) (stroke (width 0.12) (type solid)) (layer "F.SilkS"))
  (pad "1" thru_hole rect (at 0 0 180) (size 3 3) (drill 1.75) (layers "*.Cu" "*.Mask") (remove_unused_layers no) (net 33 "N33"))
  (pad "2" thru_hole circle (at 3.88 0 180) (size 3 3) (drill 1.75) (layers "*.Cu" "*.Mask") (remove_unused_layers no) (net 31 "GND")))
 (gr_rect (start 29 42.5) (end 77 76) (stroke (width 0.05) (type default)) (fill none) (layer "Edge.Cuts"))
 (segment (start 49.9075 73.9075) (end 51.4 75.4) (width 0.2) (layer "F.Cu") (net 33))
 (segment (start 37.81 61.84) (end 31.42 68.23) (width 0.2) (layer "F.Cu") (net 33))
 (segment (start 51.4 75.4) (end 63.42 75.4) (width 0.2) (layer "F.Cu") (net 33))
 (segment (start 49.9075 70.75) (end 49.9075 73.9075) (width 0.2) (layer "F.Cu") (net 33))
 (segment (start 74 67) (end 68.84 61.84) (width 0.2) (layer "F.Cu") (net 33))
 (segment (start 63.42 75.4) (end 66.5 72.32) (width 0.2) (layer "F.Cu") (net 33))
 (segment (start 49.9075 70.75) (end 51.775 70.75) (width 0.2) (layer "F.Cu") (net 33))
 (segment (start 51.775 70.75) (end 54.525 73.5) (width 0.2) (layer "F.Cu") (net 33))
 (segment (start 74 67) (end 68.68 72.32) (width 0.2) (layer "F.Cu") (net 33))
 (segment (start 68.84 61.84) (end 37.81 61.84) (width 0.2) (layer "F.Cu") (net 33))
 (segment (start 68.68 72.32) (end 66.5 72.32) (width 0.2) (layer "F.Cu") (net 33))
 (segment (start 46.0275 70.75) (end 47.8275 68.95) (width 0.2) (layer "F.Cu") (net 31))
 (segment (start 47.8275 68.95) (end 51.847244 68.95) (width 0.2) (layer "F.Cu") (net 31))
 (segment (start 51.5475 65.23) (end 56.02 65.23) (width 0.2) (layer "F.Cu") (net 31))
 (segment (start 60.96 72) (end 58.285 74.675) (width 0.2) (layer "F.Cu") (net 31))
 (segment (start 46.0275 70.75) (end 51.5475 65.23) (width 0.2) (layer "F.Cu") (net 31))
 (segment (start 53.15 67.020792) (end 53.15 65.979208) (width 0.2) (layer "F.Cu") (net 31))
 (segment (start 41.99 70.99) (end 41.99 70.64) (width 0.2) (layer "F.Cu") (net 31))
 (segment (start 56 73.102756) (end 56 73.872244) (width 0.2) (layer "F.Cu") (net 31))
 (segment (start 55.96 65) (end 55.73 65.23) (width 0.2) (layer "F.Cu") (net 31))
 (segment (start 45.3775 71.4) (end 46.0275 70.75) (width 0.2) (layer "F.Cu") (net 31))
 (segment (start 51.847244 68.95) (end 56 73.102756) (width 0.2) (layer "F.Cu") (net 31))
 (segment (start 61.915256 68.5) (end 62 68.5) (width 0.2) (layer "F.Cu") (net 31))
 (segment (start 56.802756 74.675) (end 56.4875 74.359744) (width 0.2) (layer "F.Cu") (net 31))
 (segment (start 62 68.5) (end 62 70.96) (width 0.2) (layer "F.Cu") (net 31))
 (segment (start 53.15 65.979208) (end 53.899208 65.23) (width 0.2) (layer "F.Cu") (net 31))
 (segment (start 41.58 71.4) (end 45.3775 71.4) (width 0.2) (layer "F.Cu") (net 31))
 (segment (start 53.899208 65.23) (end 56.02 65.23) (width 0.2) (layer "F.Cu") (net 31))
 (segment (start 57.127756 75) (end 57.96 75) (width 0.2) (layer "F.Cu") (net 31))
 (segment (start 62 70.96) (end 60.96 72) (width 0.2) (layer "F.Cu") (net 31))
 (segment (start 56.4875 70.358292) (end 53.15 67.020792) (width 0.2) (layer "F.Cu") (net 31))
 (segment (start 56.4875 74.359744) (end 56.4875 70.358292) (width 0.2) (layer "F.Cu") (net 31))
 (segment (start 56 73.872244) (end 57.127756 75) (width 0.2) (layer "F.Cu") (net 31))
 (segment (start 58.285 74.675) (end 56.802756 74.675) (width 0.2) (layer "F.Cu") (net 31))
 (segment (start 41.58 71.4) (end 41.99 70.99) (width 0.2) (layer "F.Cu") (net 31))
 (segment (start 57.96 75) (end 60.96 72) (width 0.2) (layer "F.Cu") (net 31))
 (segment (start 62.6 67.5) (end 62.901471 67.801471) (width 0.2) (layer "F.Cu") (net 35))
 (segment (start 62.3 72.497057) (end 63.002943 73.2) (width 0.2) (layer "F.Cu") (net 35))
 (segment (start 56.02 68.07) (end 56.02 67.77) (width 0.2) (layer "F.Cu") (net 35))
 (segment (start 57.5 73.5) (end 57.5 72.625001) (width 0.2) (layer "F.Cu") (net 35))
 (segment (start 57.5 69.25) (end 56.02 67.77) (width 0.2) (layer "F.Cu") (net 35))
 (segment (start 70.12 67) (end 66.5 70.62) (width 0.2) (layer "F.Cu") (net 35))
 (segment (start 64.780001 73.2) (end 66.300001 71.68) (width 0.2) (layer "F.Cu") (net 35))
 (segment (start 57.5 72.625001) (end 61.1 69.025001) (width 0.2) (layer "F.Cu") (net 35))
 (segment (start 57.5 73.5) (end 57.5 69.25) (width 0.2) (layer "F.Cu") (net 35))
 (segment (start 66.5 70.62) (end 66.5 71.68) (width 0.2) (layer "F.Cu") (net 35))
 (segment (start 61.1 67.815256) (end 61.415256 67.5) (width 0.2) (layer "F.Cu") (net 35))
 (segment (start 62.3 71.502943) (end 62.3 72.497057) (width 0.2) (layer "F.Cu") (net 35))
 (segment (start 61.415256 67.5) (end 62.6 67.5) (width 0.2) (layer "F.Cu") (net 35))
 (segment (start 62.901471 67.801471) (end 62.901471 70.901472) (width 0.2) (layer "F.Cu") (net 35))
 (segment (start 62.901471 70.901472) (end 62.3 71.502943) (width 0.2) (layer "F.Cu") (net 35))
 (segment (start 57.5 73.5) (end 57.7 73.7) (width 0.2) (layer "F.Cu") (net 35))
 (segment (start 63.002943 73.2) (end 64.780001 73.2) (width 0.2) (layer "F.Cu") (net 35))
 (segment (start 70.12 67.077057) (end 70.12 67) (width 0.2) (layer "F.Cu") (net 35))
 (segment (start 61.1 69.025001) (end 61.1 67.815256) (width 0.2) (layer "F.Cu") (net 35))
 (segment (start 66.300001 71.68) (end 66.5 71.68) (width 0.2) (layer "F.Cu") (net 35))
 (segment (start 63.5 65.5) (end 64.5 64.5) (width 0.2) (layer "F.Cu") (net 36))
 (segment (start 63.5 72) (end 63.5 65.5) (width 0.2) (layer "F.Cu") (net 36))
 (segment (start 61 64) (end 60 65) (width 0.2) (layer "F.Cu") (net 34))
 (segment (start 58.5 66.5) (end 54.75 66.5) (width 0.2) (layer "F.Cu") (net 34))
 (segment (start 60 65) (end 60 68.5) (width 0.2) (layer "F.Cu") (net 34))
 (segment (start 61 64) (end 58.5 66.5) (width 0.2) (layer "F.Cu") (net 34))
 (segment (start 61 64) (end 60.4 63.4) (width 0.2) (layer "F.Cu") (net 34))
 (segment (start 65.184744 63.6) (end 65.5 63.915256) (width 0.2) (layer "F.Cu") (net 32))
 (segment (start 64.584744 63) (end 66.5 63) (width 0.2) (layer "F.Cu") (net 32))
 (segment (start 61 66) (end 63.4 63.6) (width 0.2) (layer "F.Cu") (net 32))
 (segment (start 31.42 70.76) (end 31.42 70.58) (width 0.2) (layer "F.Cu") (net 32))
 (segment (start 38 62.645578) (end 38 62.24) (width 0.2) (layer "F.Cu") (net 32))
 (segment (start 66.5 64.5) (end 64.5 66.5) (width 0.2) (layer "F.Cu") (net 32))
 (segment (start 38 62.24) (end 63.824744 62.24) (width 0.2) (layer "F.Cu") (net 32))
 (segment (start 65.5 65.5) (end 64.5 66.5) (width 0.2) (layer "F.Cu") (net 32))
 (segment (start 31.42 70.76) (end 32.865 69.315) (width 0.2) (layer "F.Cu") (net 32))
 (segment (start 32.865 69.315) (end 32.865 67.780578) (width 0.2) (layer "F.Cu") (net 32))
 (segment (start 66.5 63) (end 66.5 64.5) (width 0.2) (layer "F.Cu") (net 32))
 (segment (start 63.4 63.6) (end 65.184744 63.6) (width 0.2) (layer "F.Cu") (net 32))
 (segment (start 65.5 63.915256) (end 65.5 65.5) (width 0.2) (layer "F.Cu") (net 32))
 (segment (start 32.865 67.780578) (end 38 62.645578) (width 0.2) (layer "F.Cu") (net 32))
 (segment (start 63.824744 62.24) (end 64.584744 63) (width 0.2) (layer "F.Cu") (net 32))
 (segment (start 37.17 72) (end 41.58 67.59) (width 0.2) (layer "F.Cu") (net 9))
 (segment (start 31 59.5) (end 29.5 61) (width 0.2) (layer "F.Cu") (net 9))
 (segment (start 54.58 60.74) (end 53.34 59.5) (width 0.2) (layer "F.Cu") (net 9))
 (segment (start 30.765578 72) (end 37.17 72) (width 0.2) (layer "F.Cu") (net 9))
 (segment (start 29.5 61) (end 29.5 70.734422) (width 0.2) (layer "F.Cu") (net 9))
 (segment (start 53.34 59.5) (end 31 59.5) (width 0.2) (layer "F.Cu") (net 9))
 (segment (start 29.5 70.734422) (end 30.765578 72) (width 0.2) (layer "F.Cu") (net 9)))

